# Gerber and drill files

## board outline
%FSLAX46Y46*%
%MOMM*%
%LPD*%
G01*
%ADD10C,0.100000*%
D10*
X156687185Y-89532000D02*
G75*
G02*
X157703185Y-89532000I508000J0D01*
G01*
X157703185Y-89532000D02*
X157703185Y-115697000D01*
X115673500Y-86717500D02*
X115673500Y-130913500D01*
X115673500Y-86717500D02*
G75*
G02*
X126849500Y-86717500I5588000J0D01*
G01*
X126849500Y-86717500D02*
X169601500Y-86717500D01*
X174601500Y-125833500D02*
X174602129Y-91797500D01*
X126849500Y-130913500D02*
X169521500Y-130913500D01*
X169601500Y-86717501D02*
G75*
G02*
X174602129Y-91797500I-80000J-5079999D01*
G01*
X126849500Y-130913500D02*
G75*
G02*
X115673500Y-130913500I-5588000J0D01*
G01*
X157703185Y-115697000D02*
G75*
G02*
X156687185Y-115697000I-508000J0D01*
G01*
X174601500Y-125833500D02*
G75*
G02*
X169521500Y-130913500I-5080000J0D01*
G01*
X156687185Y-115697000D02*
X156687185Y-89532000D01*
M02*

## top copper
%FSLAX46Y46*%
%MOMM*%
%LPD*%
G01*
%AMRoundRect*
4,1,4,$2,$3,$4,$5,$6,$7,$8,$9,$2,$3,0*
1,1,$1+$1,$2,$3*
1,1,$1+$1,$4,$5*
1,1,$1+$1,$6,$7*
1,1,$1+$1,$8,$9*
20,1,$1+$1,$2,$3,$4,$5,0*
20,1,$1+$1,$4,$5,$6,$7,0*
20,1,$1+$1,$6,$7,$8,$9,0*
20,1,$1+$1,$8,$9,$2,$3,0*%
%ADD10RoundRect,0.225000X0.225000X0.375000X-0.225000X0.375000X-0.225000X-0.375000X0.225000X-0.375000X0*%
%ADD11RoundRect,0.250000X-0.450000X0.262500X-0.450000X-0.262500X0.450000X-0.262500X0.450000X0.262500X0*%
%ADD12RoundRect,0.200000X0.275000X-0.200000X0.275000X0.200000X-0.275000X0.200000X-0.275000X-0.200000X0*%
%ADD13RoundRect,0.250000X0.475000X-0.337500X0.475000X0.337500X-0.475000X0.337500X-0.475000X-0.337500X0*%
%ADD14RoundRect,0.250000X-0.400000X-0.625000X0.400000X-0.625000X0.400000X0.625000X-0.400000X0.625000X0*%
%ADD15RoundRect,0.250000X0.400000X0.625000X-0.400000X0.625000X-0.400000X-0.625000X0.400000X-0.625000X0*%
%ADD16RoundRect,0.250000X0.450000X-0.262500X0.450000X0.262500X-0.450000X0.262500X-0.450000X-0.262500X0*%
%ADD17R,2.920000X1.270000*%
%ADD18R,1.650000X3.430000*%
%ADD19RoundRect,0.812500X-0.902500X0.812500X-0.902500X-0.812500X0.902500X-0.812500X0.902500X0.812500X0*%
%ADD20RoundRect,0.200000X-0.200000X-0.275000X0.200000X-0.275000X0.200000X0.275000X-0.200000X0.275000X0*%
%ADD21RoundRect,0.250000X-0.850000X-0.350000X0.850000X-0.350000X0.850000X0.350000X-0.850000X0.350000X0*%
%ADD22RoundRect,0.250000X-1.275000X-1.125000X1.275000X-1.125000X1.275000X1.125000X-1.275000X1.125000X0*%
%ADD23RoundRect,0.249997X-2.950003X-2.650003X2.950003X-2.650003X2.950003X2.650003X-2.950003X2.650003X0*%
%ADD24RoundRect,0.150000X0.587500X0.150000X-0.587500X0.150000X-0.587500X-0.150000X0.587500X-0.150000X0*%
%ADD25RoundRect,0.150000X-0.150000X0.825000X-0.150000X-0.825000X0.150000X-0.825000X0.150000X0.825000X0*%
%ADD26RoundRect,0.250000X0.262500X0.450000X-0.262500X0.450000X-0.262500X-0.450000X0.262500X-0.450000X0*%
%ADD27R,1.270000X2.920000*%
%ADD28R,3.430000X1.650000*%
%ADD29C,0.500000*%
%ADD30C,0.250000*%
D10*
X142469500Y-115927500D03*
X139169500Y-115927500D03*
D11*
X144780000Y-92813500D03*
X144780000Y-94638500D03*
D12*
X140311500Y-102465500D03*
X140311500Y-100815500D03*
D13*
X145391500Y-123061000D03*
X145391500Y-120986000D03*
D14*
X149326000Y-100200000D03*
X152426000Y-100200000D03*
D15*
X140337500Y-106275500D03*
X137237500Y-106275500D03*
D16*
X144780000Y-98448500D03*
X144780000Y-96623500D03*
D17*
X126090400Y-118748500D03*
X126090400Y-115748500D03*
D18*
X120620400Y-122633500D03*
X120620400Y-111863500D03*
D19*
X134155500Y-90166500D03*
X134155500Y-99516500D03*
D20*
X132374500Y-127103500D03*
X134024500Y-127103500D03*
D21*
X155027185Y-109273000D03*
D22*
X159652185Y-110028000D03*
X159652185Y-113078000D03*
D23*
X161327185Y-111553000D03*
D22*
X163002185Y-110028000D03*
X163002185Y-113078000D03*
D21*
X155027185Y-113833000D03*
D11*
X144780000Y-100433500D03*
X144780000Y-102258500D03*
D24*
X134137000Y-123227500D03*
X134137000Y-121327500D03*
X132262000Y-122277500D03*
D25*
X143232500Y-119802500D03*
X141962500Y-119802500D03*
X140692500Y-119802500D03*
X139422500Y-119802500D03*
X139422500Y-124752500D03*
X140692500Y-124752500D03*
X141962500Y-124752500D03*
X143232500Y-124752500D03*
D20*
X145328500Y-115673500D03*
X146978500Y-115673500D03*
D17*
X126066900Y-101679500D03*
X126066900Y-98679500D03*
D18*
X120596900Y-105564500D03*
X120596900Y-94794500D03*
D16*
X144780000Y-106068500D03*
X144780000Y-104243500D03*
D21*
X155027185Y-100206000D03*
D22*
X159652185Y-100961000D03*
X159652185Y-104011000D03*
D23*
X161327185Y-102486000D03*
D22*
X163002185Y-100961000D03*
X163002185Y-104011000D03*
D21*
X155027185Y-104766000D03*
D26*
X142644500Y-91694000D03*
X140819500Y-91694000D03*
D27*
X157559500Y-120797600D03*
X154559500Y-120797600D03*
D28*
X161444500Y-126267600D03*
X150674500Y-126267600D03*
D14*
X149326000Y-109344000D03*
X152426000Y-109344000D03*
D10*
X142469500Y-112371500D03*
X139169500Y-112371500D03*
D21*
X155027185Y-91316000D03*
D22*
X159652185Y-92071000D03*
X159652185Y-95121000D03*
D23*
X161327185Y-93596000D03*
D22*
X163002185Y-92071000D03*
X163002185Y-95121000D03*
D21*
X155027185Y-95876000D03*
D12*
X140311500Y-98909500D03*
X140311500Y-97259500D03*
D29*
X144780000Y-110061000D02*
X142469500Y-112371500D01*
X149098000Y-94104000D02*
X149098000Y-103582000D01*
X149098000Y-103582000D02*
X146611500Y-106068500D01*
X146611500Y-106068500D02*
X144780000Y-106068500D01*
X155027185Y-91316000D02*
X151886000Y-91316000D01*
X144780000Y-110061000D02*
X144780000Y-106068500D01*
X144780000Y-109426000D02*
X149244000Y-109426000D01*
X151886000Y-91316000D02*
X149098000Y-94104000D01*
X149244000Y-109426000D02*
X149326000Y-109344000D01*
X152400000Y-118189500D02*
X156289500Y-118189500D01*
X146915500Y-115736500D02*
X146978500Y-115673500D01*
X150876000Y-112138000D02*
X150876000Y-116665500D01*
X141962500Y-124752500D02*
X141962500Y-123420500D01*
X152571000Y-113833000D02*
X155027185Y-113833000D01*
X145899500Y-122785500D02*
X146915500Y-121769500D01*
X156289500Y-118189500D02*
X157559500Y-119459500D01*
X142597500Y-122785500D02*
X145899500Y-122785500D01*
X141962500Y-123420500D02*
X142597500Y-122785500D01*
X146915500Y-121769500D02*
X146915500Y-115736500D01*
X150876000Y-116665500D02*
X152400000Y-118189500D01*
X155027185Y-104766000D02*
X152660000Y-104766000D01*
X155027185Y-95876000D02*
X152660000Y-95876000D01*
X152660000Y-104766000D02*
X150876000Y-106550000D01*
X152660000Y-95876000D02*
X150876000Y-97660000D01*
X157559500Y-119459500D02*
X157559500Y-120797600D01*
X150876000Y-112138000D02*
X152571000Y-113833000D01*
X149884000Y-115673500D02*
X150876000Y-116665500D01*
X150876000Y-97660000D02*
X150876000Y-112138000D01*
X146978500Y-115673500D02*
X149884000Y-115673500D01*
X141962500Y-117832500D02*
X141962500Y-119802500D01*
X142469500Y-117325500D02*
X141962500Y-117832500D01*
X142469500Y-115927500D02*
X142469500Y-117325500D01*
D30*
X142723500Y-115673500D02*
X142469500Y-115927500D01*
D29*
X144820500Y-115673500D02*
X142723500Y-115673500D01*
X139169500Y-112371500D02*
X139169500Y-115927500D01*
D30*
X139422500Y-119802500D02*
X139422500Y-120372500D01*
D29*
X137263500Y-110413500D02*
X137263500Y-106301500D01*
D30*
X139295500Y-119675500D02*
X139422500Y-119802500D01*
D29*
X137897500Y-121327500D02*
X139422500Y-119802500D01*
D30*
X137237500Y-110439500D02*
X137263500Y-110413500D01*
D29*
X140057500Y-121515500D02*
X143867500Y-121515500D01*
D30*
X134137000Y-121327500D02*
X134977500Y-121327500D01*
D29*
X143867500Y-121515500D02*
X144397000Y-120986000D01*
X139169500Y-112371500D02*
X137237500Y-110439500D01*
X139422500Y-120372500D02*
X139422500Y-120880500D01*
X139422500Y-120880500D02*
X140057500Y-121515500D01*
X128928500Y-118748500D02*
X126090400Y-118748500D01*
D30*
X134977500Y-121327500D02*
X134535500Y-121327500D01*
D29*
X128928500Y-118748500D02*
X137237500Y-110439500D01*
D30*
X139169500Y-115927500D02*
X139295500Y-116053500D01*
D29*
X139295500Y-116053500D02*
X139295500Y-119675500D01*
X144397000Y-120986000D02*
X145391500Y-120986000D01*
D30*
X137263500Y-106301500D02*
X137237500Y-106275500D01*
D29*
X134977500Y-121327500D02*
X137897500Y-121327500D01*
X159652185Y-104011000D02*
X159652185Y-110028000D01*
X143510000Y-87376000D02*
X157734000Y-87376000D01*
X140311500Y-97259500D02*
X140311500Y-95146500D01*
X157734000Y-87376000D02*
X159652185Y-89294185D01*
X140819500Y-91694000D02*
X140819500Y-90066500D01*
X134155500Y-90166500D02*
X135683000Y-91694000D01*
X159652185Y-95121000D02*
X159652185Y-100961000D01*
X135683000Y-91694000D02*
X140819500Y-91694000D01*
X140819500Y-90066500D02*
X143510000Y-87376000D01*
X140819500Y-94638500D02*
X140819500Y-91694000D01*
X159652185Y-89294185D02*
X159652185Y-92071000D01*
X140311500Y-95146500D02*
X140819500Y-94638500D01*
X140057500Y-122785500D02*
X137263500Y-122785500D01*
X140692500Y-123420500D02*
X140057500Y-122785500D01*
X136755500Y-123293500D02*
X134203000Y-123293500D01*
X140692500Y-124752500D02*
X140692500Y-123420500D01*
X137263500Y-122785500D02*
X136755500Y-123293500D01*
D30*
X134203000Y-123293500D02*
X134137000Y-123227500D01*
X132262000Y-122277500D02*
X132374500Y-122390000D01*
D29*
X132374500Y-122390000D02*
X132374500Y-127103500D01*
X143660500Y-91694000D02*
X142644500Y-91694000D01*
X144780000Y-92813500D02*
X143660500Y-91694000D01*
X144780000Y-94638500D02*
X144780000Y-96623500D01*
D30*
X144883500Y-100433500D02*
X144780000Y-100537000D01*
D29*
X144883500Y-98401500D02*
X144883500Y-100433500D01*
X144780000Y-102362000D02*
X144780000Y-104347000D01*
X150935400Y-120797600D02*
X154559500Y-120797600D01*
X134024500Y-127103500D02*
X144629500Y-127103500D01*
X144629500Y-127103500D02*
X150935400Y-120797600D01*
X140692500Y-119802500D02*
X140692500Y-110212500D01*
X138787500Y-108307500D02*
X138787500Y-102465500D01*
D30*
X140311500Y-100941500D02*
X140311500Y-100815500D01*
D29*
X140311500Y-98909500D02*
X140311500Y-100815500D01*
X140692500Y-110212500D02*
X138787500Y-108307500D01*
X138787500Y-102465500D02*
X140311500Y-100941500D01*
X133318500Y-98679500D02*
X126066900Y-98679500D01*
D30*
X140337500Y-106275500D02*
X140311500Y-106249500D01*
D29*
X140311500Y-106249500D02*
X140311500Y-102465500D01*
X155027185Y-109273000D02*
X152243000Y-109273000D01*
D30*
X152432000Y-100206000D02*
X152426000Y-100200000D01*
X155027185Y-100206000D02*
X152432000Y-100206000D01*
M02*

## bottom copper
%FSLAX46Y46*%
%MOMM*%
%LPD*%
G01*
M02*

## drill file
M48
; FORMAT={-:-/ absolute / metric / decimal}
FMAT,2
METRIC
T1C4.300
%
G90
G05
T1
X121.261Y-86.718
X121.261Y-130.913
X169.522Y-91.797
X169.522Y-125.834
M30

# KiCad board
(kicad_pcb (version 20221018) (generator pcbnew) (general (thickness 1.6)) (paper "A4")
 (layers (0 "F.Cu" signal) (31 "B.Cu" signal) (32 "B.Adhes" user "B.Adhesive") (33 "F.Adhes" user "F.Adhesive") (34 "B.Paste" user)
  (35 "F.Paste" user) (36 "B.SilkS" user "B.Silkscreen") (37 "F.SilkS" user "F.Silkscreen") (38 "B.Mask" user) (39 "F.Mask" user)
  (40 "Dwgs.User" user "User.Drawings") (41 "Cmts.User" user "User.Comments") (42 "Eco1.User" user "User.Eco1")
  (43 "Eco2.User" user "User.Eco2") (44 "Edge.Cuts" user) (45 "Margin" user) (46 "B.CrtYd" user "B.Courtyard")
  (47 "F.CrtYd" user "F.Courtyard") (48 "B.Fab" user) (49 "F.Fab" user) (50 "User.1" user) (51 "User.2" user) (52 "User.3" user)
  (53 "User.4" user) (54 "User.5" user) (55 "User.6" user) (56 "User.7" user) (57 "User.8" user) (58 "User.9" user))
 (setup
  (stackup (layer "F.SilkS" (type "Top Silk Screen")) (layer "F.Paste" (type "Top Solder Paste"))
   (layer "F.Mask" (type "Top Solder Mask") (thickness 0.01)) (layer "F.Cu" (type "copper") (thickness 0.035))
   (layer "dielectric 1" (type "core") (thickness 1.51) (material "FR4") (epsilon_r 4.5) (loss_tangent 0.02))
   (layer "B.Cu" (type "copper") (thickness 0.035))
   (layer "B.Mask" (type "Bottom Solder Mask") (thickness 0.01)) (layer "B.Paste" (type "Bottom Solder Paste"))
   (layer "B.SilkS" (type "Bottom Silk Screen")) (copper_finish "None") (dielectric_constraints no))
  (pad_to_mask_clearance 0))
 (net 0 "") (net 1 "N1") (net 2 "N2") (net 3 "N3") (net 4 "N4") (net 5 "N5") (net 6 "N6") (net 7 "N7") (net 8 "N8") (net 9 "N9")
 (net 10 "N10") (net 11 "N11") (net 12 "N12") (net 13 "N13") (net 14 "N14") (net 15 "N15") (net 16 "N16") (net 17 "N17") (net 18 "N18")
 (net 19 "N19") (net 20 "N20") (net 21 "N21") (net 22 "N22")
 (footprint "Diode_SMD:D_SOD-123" (layer "F.Cu") (at 140.8195 115.9275 180)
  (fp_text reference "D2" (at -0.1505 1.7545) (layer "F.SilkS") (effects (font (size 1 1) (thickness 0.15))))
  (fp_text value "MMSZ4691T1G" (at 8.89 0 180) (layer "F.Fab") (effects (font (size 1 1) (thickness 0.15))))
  (pad "1" smd roundrect (at -1.65 0 180) (size 0.9 1.2) (layers "F.Cu" "F.Paste" "F.Mask") (roundrect_rratio 0.25) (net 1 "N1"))
  (pad "2" smd roundrect (at 1.65 0 180) (size 0.9 1.2) (layers "F.Cu" "F.Paste" "F.Mask") (roundrect_rratio 0.25) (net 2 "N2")))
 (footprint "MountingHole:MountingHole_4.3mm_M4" (layer "F.Cu") (at 169.5215 91.7975)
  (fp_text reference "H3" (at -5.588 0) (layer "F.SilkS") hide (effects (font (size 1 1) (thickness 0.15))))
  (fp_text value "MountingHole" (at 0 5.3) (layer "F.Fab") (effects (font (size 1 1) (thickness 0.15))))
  (pad "" np_thru_hole circle (at 0 0) (size 4.3 4.3) (drill 4.3) (layers "*.Cu" "*.Mask")))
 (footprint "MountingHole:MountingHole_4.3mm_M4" (layer "F.Cu") (at 121.2615 130.9135)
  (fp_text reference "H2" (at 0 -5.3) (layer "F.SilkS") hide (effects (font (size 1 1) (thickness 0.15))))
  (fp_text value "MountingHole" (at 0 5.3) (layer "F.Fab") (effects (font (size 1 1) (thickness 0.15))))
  (pad "" np_thru_hole circle (at 0 0) (size 4.3 4.3) (drill 4.3) (layers "*.Cu" "*.Mask")))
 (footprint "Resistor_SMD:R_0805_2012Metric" (layer "F.Cu") (at 144.78 93.726 -90)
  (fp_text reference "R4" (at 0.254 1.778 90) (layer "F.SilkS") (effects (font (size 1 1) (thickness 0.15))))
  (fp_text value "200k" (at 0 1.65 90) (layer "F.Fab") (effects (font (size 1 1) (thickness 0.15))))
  (pad "1" smd roundrect (at -0.9125 0 270) (size 1.025 1.4) (layers "F.Cu" "F.Paste" "F.Mask") (roundrect_rratio 0.243902) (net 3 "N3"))
  (pad "2" smd roundrect (at 0.9125 0 270) (size 1.025 1.4) (layers "F.Cu" "F.Paste" "F.Mask") (roundrect_rratio 0.243902) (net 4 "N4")))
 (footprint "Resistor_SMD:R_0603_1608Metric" (layer "F.Cu") (at 140.3115 101.6405 90)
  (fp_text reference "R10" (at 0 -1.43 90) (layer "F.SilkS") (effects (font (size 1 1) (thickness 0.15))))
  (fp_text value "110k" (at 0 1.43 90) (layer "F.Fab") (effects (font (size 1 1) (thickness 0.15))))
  (pad "1" smd roundrect (at -0.825 0 90) (size 0.8 0.95) (layers "F.Cu" "F.Paste" "F.Mask") (roundrect_rratio 0.25) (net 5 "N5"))
  (pad "2" smd roundrect (at 0.825 0 90) (size 0.8 0.95) (layers "F.Cu" "F.Paste" "F.Mask") (roundrect_rratio 0.25) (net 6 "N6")))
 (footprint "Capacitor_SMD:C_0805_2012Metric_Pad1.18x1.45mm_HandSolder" (layer "F.Cu") (at 145.3915 122.0235 90)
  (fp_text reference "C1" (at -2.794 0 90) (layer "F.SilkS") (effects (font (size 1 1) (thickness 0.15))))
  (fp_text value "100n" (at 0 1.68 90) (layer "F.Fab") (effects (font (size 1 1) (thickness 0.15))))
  (pad "1" smd roundrect (at -1.0375 0 90) (size 1.175 1.45) (layers "F.Cu" "F.Paste" "F.Mask") (roundrect_rratio 0.212766) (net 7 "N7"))
  (pad "2" smd roundrect (at 1.0375 0 90) (size 1.175 1.45) (layers "F.Cu" "F.Paste" "F.Mask") (roundrect_rratio 0.212766) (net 2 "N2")))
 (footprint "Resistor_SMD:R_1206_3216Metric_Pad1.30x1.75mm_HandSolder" (layer "F.Cu") (at 150.876 100.2)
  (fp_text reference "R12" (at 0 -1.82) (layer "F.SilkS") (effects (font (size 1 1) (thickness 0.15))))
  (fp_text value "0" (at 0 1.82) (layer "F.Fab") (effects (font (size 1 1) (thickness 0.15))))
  (pad "1" smd roundrect (at -1.55 0) (size 1.3 1.75) (layers "F.Cu" "F.Paste" "F.Mask") (roundrect_rratio 0.192308) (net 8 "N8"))
  (pad "2" smd roundrect (at 1.55 0) (size 1.3 1.75) (layers "F.Cu" "F.Paste" "F.Mask") (roundrect_rratio 0.192308) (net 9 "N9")))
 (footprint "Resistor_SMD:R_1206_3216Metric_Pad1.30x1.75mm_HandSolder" (layer "F.Cu") (at 138.7875 106.2755 180)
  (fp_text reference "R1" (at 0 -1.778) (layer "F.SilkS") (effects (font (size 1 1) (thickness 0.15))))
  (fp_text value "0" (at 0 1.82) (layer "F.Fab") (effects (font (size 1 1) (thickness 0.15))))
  (pad "1" smd roundrect (at -1.55 0 180) (size 1.3 1.75) (layers "F.Cu" "F.Paste" "F.Mask") (roundrect_rratio 0.192308) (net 5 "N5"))
  (pad "2" smd roundrect (at 1.55 0 180) (size 1.3 1.75) (layers "F.Cu" "F.Paste" "F.Mask") (roundrect_rratio 0.192308) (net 2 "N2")))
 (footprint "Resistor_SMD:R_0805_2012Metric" (layer "F.Cu") (at 144.78 97.536 90)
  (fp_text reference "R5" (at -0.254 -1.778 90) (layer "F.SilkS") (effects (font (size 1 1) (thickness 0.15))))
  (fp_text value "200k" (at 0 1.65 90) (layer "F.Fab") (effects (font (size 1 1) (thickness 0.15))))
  (pad "1" smd roundrect (at -0.9125 0 90) (size 1.025 1.4) (layers "F.Cu" "F.Paste" "F.Mask") (roundrect_rratio 0.243902) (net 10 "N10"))
  (pad "2" smd roundrect (at 0.9125 0 90) (size 1.025 1.4) (layers "F.Cu" "F.Paste" "F.Mask") (roundrect_rratio 0.243902) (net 4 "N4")))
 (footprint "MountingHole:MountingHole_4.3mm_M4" (layer "F.Cu") (at 169.5215 125.8335)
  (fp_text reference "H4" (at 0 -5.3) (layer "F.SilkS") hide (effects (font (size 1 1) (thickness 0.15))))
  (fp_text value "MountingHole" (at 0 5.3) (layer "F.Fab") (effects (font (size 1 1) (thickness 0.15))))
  (pad "" np_thru_hole circle (at 0 0) (size 4.3 4.3) (drill 4.3) (layers "*.Cu" "*.Mask")))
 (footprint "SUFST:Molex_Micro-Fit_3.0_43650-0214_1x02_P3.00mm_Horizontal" (layer "F.Cu") (at 126.0904 117.2485 -90)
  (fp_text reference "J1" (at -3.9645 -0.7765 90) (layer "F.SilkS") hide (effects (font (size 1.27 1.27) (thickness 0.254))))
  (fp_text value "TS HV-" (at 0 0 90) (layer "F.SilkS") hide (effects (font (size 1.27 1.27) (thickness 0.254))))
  (pad "1" smd rect (at 1.5 0 270) (size 1.27 2.92) (layers "F.Cu" "F.Paste" "F.Mask") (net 2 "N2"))
  (pad "2" smd rect (at -1.5 0 270) (size 1.27 2.92) (layers "F.Cu" "F.Paste" "F.Mask") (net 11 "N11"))
  (pad "3" smd rect (at 5.385 5.47) (size 1.65 3.43) (layers "F.Cu" "F.Paste" "F.Mask"))
  (pad "4" smd rect (at -5.385 5.47) (size 1.65 3.43) (layers "F.Cu" "F.Paste" "F.Mask")))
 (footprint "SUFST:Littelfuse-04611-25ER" (layer "F.Cu") (at 134.2155 94.5915 -90)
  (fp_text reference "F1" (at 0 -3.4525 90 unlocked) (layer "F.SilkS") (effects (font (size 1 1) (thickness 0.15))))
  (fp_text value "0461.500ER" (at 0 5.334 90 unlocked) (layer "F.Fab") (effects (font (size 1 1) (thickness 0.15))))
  (pad "1" smd roundrect (at -4.425 0.06 270) (size 3.25 3.43) (layers "F.Cu" "F.Paste" "F.Mask") (roundrect_rratio 0.25) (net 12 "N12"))
  (pad "2" smd roundrect (at 4.925 0.06 270) (size 3.25 3.43) (layers "F.Cu" "F.Paste" "F.Mask") (roundrect_rratio 0.25) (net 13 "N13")))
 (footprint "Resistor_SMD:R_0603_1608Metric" (layer "F.Cu") (at 133.1995 127.1035)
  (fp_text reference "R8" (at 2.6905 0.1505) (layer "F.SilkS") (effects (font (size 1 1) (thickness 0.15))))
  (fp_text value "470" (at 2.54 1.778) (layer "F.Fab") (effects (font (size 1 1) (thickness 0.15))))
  (pad "1" smd roundrect (at -0.825 0) (size 0.8 0.95) (layers "F.Cu" "F.Paste" "F.Mask") (roundrect_rratio 0.25) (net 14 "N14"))
  (pad "2" smd roundrect (at 0.825 0) (size 0.8 0.95) (layers "F.Cu" "F.Paste" "F.Mask") (roundrect_rratio 0.25) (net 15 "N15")))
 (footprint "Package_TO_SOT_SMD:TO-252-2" (layer "F.Cu") (at 160.067185 111.553)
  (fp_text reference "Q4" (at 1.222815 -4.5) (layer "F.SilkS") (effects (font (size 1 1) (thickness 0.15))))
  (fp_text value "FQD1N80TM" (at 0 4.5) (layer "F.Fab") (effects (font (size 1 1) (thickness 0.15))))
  (pad "1" smd roundrect (at -5.04 -2.28) (size 2.2 1.2) (layers "F.Cu" "F.Paste" "F.Mask") (roundrect_rratio 0.208333) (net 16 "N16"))
  (pad "2" smd roundrect (at -0.415 -1.525) (size 3.05 2.75) (layers "F.Cu" "F.Paste") (roundrect_rratio 0.090909) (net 12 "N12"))
  (pad "2" smd roundrect (at -0.415 1.525) (size 3.05 2.75) (layers "F.Cu" "F.Paste") (roundrect_rratio 0.090909) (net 12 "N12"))
  (pad "2" smd roundrect (at 1.26 0) (size 6.4 5.8) (layers "F.Cu" "F.Mask") (roundrect_rratio 0.043103) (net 12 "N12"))
  (pad "2" smd roundrect (at 2.935 -1.525) (size 3.05 2.75) (layers "F.Cu" "F.Paste") (roundrect_rratio 0.090909) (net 12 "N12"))
  (pad "2" smd roundrect (at 2.935 1.525) (size 3.05 2.75) (layers "F.Cu" "F.Paste") (roundrect_rratio 0.090909) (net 12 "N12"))
  (pad "3" smd roundrect (at -5.04 2.28) (size 2.2 1.2) (layers "F.Cu" "F.Paste" "F.Mask") (roundrect_rratio 0.208333) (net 7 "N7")))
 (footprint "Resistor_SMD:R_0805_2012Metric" (layer "F.Cu") (at 144.78 101.346 -90)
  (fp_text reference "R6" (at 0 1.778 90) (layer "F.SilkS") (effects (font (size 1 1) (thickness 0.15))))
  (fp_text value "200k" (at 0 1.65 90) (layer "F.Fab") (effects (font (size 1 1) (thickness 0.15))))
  (pad "1" smd roundrect (at -0.9125 0 270) (size 1.025 1.4) (layers "F.Cu" "F.Paste" "F.Mask") (roundrect_rratio 0.243902) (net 10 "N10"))
  (pad "2" smd roundrect (at 0.9125 0 270) (size 1.025 1.4) (layers "F.Cu" "F.Paste" "F.Mask") (roundrect_rratio 0.243902) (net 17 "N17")))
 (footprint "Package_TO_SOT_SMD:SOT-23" (layer "F.Cu") (at 133.1995 122.2775 180)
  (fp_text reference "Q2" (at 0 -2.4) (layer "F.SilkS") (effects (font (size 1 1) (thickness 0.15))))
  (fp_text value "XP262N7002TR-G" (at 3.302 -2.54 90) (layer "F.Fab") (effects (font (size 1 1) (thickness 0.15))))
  (pad "1" smd roundrect (at -0.9375 -0.95 180) (size 1.475 0.6) (layers "F.Cu" "F.Paste" "F.Mask") (roundrect_rratio 0.25) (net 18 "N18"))
  (pad "2" smd roundrect (at -0.9375 0.95 180) (size 1.475 0.6) (layers "F.Cu" "F.Paste" "F.Mask") (roundrect_rratio 0.25) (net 2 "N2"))
  (pad "3" smd roundrect (at 0.9375 0 180) (size 1.475 0.6) (layers "F.Cu" "F.Paste" "F.Mask") (roundrect_rratio 0.25) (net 14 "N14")))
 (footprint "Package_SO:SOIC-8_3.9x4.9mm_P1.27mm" (layer "F.Cu") (at 141.3275 122.2775 -90)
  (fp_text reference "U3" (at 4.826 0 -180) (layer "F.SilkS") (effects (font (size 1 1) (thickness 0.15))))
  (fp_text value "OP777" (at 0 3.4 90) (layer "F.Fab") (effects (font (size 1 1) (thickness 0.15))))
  (pad "1" smd roundrect (at -2.475 -1.905 270) (size 1.95 0.6) (layers "F.Cu" "F.Paste" "F.Mask") (roundrect_rratio 0.25) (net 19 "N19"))
  (pad "2" smd roundrect (at -2.475 -0.635 270) (size 1.95 0.6) (layers "F.Cu" "F.Paste" "F.Mask") (roundrect_rratio 0.25) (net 1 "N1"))
  (pad "3" smd roundrect (at -2.475 0.635 270) (size 1.95 0.6) (layers "F.Cu" "F.Paste" "F.Mask") (roundrect_rratio 0.25) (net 6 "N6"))
  (pad "4" smd roundrect (at -2.475 1.905 270) (size 1.95 0.6) (layers "F.Cu" "F.Paste" "F.Mask") (roundrect_rratio 0.25) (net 2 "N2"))
  (pad "5" smd roundrect (at 2.475 1.905 270) (size 1.95 0.6) (layers "F.Cu" "F.Paste" "F.Mask") (roundrect_rratio 0.25) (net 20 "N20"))
  (pad "6" smd roundrect (at 2.475 0.635 270) (size 1.95 0.6) (layers "F.Cu" "F.Paste" "F.Mask") (roundrect_rratio 0.25) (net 18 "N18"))
  (pad "7" smd roundrect (at 2.475 -0.635 270) (size 1.95 0.6) (layers "F.Cu" "F.Paste" "F.Mask") (roundrect_rratio 0.25) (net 7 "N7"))
  (pad "8" smd roundrect (at 2.475 -1.905 270) (size 1.95 0.6) (layers "F.Cu" "F.Paste" "F.Mask") (roundrect_rratio 0.25) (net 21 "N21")))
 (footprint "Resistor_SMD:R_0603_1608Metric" (layer "F.Cu") (at 146.1535 115.6735)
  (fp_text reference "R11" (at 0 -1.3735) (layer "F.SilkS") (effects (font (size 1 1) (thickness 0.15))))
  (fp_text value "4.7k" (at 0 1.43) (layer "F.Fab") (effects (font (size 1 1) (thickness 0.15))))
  (pad "1" smd roundrect (at -0.825 0) (size 0.8 0.95) (layers "F.Cu" "F.Paste" "F.Mask") (roundrect_rratio 0.25) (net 1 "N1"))
  (pad "2" smd roundrect (at 0.825 0) (size 0.8 0.95) (layers "F.Cu" "F.Paste" "F.Mask") (roundrect_rratio 0.25) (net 7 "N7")))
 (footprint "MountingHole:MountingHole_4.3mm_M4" (layer "F.Cu") (at 121.2615 86.7175)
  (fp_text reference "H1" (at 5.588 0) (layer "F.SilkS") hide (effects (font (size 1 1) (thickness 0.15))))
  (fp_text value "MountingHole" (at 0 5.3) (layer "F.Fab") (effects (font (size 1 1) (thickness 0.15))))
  (pad "" np_thru_hole circle (at 0 0) (size 4.3 4.3) (drill 4.3) (layers "*.Cu" "*.Mask")))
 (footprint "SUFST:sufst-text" (layer "F.Cu") (at 168.402 108.712 90)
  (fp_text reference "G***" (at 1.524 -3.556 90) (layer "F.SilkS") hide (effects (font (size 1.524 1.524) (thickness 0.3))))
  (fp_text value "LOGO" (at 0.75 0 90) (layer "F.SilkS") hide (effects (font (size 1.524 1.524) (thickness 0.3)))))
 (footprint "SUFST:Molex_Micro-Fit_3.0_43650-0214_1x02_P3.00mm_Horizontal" (layer "F.Cu") (at 126.0669 100.1795 -90)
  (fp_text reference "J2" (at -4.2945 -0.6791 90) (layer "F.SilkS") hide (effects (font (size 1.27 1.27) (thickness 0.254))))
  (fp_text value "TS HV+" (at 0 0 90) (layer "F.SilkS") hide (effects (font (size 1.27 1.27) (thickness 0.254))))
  (pad "1" smd rect (at 1.5 0 270) (size 1.27 2.92) (layers "F.Cu" "F.Paste" "F.Mask") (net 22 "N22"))
  (pad "2" smd rect (at -1.5 0 270) (size 1.27 2.92) (layers "F.Cu" "F.Paste" "F.Mask") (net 13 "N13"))
  (pad "3" smd rect (at 5.385 5.47) (size 1.65 3.43) (layers "F.Cu" "F.Paste" "F.Mask"))
  (pad "4" smd rect (at -5.385 5.47) (size 1.65 3.43) (layers "F.Cu" "F.Paste" "F.Mask")))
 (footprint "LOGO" (layer "F.Cu") (at 131.064 113.792 90)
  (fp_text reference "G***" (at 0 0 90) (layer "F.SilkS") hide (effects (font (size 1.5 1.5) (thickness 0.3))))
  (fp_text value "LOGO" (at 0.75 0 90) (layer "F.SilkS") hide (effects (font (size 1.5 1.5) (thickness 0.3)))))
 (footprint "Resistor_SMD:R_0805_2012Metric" (layer "F.Cu") (at 144.78 105.156 90)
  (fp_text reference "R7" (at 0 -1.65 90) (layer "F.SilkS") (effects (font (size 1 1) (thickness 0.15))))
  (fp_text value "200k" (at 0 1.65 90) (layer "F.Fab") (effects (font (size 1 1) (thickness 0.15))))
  (pad "1" smd roundrect (at -0.9125 0 90) (size 1.025 1.4) (layers "F.Cu" "F.Paste" "F.Mask") (roundrect_rratio 0.243902) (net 8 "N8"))
  (pad "2" smd roundrect (at 0.9125 0 90) (size 1.025 1.4) (layers "F.Cu" "F.Paste" "F.Mask") (roundrect_rratio 0.243902) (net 17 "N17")))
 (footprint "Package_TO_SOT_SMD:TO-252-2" (layer "F.Cu") (at 160.067185 102.486)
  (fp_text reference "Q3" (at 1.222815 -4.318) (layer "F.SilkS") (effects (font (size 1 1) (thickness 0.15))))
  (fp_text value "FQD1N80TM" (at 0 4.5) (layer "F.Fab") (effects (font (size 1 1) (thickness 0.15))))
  (pad "1" smd roundrect (at -5.04 -2.28) (size 2.2 1.2) (layers "F.Cu" "F.Paste" "F.Mask") (roundrect_rratio 0.208333) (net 9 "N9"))
  (pad "2" smd roundrect (at -0.415 -1.525) (size 3.05 2.75) (layers "F.Cu" "F.Paste") (roundrect_rratio 0.090909) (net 12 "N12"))
  (pad "2" smd roundrect (at -0.415 1.525) (size 3.05 2.75) (layers "F.Cu" "F.Paste") (roundrect_rratio 0.090909) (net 12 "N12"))
  (pad "2" smd roundrect (at 1.26 0) (size 6.4 5.8) (layers "F.Cu" "F.Mask") (roundrect_rratio 0.043103) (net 12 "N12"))
  (pad "2" smd roundrect (at 2.935 -1.525) (size 3.05 2.75) (layers "F.Cu" "F.Paste") (roundrect_rratio 0.090909) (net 12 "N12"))
  (pad "2" smd roundrect (at 2.935 1.525) (size 3.05 2.75) (layers "F.Cu" "F.Paste") (roundrect_rratio 0.090909) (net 12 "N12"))
  (pad "3" smd roundrect (at -5.04 2.28) (size 2.2 1.2) (layers "F.Cu" "F.Paste" "F.Mask") (roundrect_rratio 0.208333) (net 7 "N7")))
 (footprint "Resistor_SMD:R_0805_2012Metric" (layer "F.Cu") (at 141.732 91.694 180)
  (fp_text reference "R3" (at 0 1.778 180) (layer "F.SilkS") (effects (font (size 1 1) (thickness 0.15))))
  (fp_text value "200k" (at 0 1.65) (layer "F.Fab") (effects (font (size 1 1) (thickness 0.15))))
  (pad "1" smd roundrect (at -0.9125 0 180) (size 1.025 1.4) (layers "F.Cu" "F.Paste" "F.Mask") (roundrect_rratio 0.243902) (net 3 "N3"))
  (pad "2" smd roundrect (at 0.9125 0 180) (size 1.025 1.4) (layers "F.Cu" "F.Paste" "F.Mask") (roundrect_rratio 0.243902) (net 12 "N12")))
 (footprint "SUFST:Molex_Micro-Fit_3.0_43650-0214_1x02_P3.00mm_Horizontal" (layer "F.Cu") (at 156.0595 120.7976)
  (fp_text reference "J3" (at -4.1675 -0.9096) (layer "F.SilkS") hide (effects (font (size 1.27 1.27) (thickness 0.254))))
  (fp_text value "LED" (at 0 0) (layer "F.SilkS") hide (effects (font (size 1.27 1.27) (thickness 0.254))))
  (pad "1" smd rect (at 1.5 0) (size 1.27 2.92) (layers "F.Cu" "F.Paste" "F.Mask") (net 7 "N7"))
  (pad "2" smd rect (at -1.5 0) (size 1.27 2.92) (layers "F.Cu" "F.Paste" "F.Mask") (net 15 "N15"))
  (pad "3" smd rect (at 5.385 5.47 90) (size 1.65 3.43) (layers "F.Cu" "F.Paste" "F.Mask"))
  (pad "4" smd rect (at -5.385 5.47 90) (size 1.65 3.43) (layers "F.Cu" "F.Paste" "F.Mask")))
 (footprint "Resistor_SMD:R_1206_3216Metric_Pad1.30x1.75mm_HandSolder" (layer "F.Cu") (at 150.876 109.344)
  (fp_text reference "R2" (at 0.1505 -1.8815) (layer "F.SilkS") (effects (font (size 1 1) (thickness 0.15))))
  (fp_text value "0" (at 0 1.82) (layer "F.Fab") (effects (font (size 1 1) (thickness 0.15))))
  (pad "1" smd roundrect (at -1.55 0) (size 1.3 1.75) (layers "F.Cu" "F.Paste" "F.Mask") (roundrect_rratio 0.192308) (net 8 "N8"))
  (pad "2" smd roundrect (at 1.55 0) (size 1.3 1.75) (layers "F.Cu" "F.Paste" "F.Mask") (roundrect_rratio 0.192308) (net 16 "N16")))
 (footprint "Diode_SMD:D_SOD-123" (layer "F.Cu") (at 140.8195 112.3715 180)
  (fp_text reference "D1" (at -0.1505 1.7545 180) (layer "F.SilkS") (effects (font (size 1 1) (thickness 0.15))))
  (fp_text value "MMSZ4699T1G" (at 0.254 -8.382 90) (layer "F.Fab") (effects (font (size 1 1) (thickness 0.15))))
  (pad "1" smd roundrect (at -1.65 0 180) (size 0.9 1.2) (layers "F.Cu" "F.Paste" "F.Mask") (roundrect_rratio 0.25) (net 8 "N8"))
  (pad "2" smd roundrect (at 1.65 0 180) (size 0.9 1.2) (layers "F.Cu" "F.Paste" "F.Mask") (roundrect_rratio 0.25) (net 2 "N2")))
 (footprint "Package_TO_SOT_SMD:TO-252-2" (layer "F.Cu") (at 160.067185 93.596)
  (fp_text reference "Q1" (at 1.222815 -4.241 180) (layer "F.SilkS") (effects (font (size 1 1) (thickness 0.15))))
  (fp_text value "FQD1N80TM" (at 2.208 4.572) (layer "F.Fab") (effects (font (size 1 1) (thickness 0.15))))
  (pad "1" smd roundrect (at -5.04 -2.28) (size 2.2 1.2) (layers "F.Cu" "F.Paste" "F.Mask") (roundrect_rratio 0.208333) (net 8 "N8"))
  (pad "2" smd roundrect (at -0.415 -1.525) (size 3.05 2.75) (layers "F.Cu" "F.Paste") (roundrect_rratio 0.090909) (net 12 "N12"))
  (pad "2" smd roundrect (at -0.415 1.525) (size 3.05 2.75) (layers "F.Cu" "F.Paste") (roundrect_rratio 0.090909) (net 12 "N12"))
  (pad "2" smd roundrect (at 1.26 0) (size 6.4 5.8) (layers "F.Cu" "F.Mask") (roundrect_rratio 0.043103) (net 12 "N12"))
  (pad "2" smd roundrect (at 2.935 -1.525) (size 3.05 2.75) (layers "F.Cu" "F.Paste") (roundrect_rratio 0.090909) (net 12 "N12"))
  (pad "2" smd roundrect (at 2.935 1.525) (size 3.05 2.75) (layers "F.Cu" "F.Paste") (roundrect_rratio 0.090909) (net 12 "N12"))
  (pad "3" smd roundrect (at -5.04 2.28) (size 2.2 1.2) (layers "F.Cu" "F.Paste" "F.Mask") (roundrect_rratio 0.208333) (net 7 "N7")))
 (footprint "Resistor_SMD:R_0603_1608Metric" (layer "F.Cu") (at 140.3115 98.0845 90)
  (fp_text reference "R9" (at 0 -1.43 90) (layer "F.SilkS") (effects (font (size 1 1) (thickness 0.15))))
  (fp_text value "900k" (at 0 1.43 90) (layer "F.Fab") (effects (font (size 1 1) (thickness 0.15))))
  (pad "1" smd roundrect (at -0.825 0 90) (size 0.8 0.95) (layers "F.Cu" "F.Paste" "F.Mask") (roundrect_rratio 0.25) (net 6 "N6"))
  (pad "2" smd roundrect (at 0.825 0 90) (size 0.8 0.95) (layers "F.Cu" "F.Paste" "F.Mask") (roundrect_rratio 0.25) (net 12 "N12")))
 (gr_arc (start 156.687185 89.532) (mid 157.195185 89.024) (end 157.703185 89.532) (stroke (width 0.1) (type default)) (layer "Edge.Cuts"))
 (gr_line (start 157.703185 89.532) (end 157.703185 115.697) (stroke (width 0.1) (type default)) (layer "Edge.Cuts"))
 (gr_line (start 115.6735 86.7175) (end 115.6735 130.9135) (stroke (width 0.1) (type default)) (layer "Edge.Cuts"))
 (gr_arc (start 115.6735 86.7175) (mid 121.2615 81.1295) (end 126.8495 86.7175) (stroke (width 0.1) (type default)) (layer "Edge.Cuts"))
 (gr_line (start 126.8495 86.7175) (end 169.6015 86.7175) (stroke (width 0.1) (type default)) (layer "Edge.Cuts"))
 (gr_line (start 174.6015 125.8335) (end 174.602129 91.7975) (stroke (width 0.1) (type default)) (layer "Edge.Cuts"))
 (gr_line (start 126.8495 130.9135) (end 169.5215 130.9135) (stroke (width 0.1) (type default)) (layer "Edge.Cuts"))
 (gr_arc (start 169.6015 86.717501) (mid 173.142221 88.233349) (end 174.602129 91.7975) (stroke (width 0.1) (type default))
  (layer "Edge.Cuts"))
 (gr_arc (start 126.8495 130.9135) (mid 121.2615 136.5015) (end 115.6735 130.9135) (stroke (width 0.1) (type default)) (layer "Edge.Cuts"))
 (gr_arc (start 157.703185 115.697) (mid 157.195185 116.205) (end 156.687185 115.697) (stroke (width 0.1) (type default))
  (layer "Edge.Cuts"))
 (gr_arc (start 174.6015 125.8335) (mid 173.113602 129.425602) (end 169.5215 130.9135) (stroke (width 0.1) (type default))
  (layer "Edge.Cuts"))
 (gr_line (start 156.687185 115.697) (end 156.687185 89.532) (stroke (width 0.1) (type default)) (layer "Edge.Cuts"))
 (segment (start 144.78 110.061) (end 142.4695 112.3715) (width 0.5) (layer "F.Cu") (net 8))
 (segment (start 149.098 94.104) (end 149.098 103.582) (width 0.5) (layer "F.Cu") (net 8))
 (segment (start 149.098 103.582) (end 146.6115 106.0685) (width 0.5) (layer "F.Cu") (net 8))
 (segment (start 146.6115 106.0685) (end 144.78 106.0685) (width 0.5) (layer "F.Cu") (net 8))
 (segment (start 155.027185 91.316) (end 151.886 91.316) (width 0.5) (layer "F.Cu") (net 8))
 (segment (start 144.78 110.061) (end 144.78 106.0685) (width 0.5) (layer "F.Cu") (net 8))
 (segment (start 144.78 109.426) (end 149.244 109.426) (width 0.5) (layer "F.Cu") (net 8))
 (segment (start 151.886 91.316) (end 149.098 94.104) (width 0.5) (layer "F.Cu") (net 8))
 (segment (start 149.244 109.426) (end 149.326 109.344) (width 0.5) (layer "F.Cu") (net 8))
 (segment (start 152.4 118.1895) (end 156.2895 118.1895) (width 0.5) (layer "F.Cu") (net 7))
 (segment (start 146.9155 115.7365) (end 146.9785 115.6735) (width 0.5) (layer "F.Cu") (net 7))
 (segment (start 150.876 112.138) (end 150.876 116.6655) (width 0.5) (layer "F.Cu") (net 7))
 (segment (start 141.9625 124.7525) (end 141.9625 123.4205) (width 0.5) (layer "F.Cu") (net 7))
 (segment (start 152.571 113.833) (end 155.027185 113.833) (width 0.5) (layer "F.Cu") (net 7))
 (segment (start 145.8995 122.7855) (end 146.9155 121.7695) (width 0.5) (layer "F.Cu") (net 7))
 (segment (start 156.2895 118.1895) (end 157.5595 119.4595) (width 0.5) (layer "F.Cu") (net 7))
 (segment (start 142.5975 122.7855) (end 145.8995 122.7855) (width 0.5) (layer "F.Cu") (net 7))
 (segment (start 141.9625 123.4205) (end 142.5975 122.7855) (width 0.5) (layer "F.Cu") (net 7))
 (segment (start 146.9155 121.7695) (end 146.9155 115.7365) (width 0.5) (layer "F.Cu") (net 7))
 (segment (start 150.876 116.6655) (end 152.4 118.1895) (width 0.5) (layer "F.Cu") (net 7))
 (segment (start 155.027185 104.766) (end 152.66 104.766) (width 0.5) (layer "F.Cu") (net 7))
 (segment (start 155.027185 95.876) (end 152.66 95.876) (width 0.5) (layer "F.Cu") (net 7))
 (segment (start 152.66 104.766) (end 150.876 106.55) (width 0.5) (layer "F.Cu") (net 7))
 (segment (start 152.66 95.876) (end 150.876 97.66) (width 0.5) (layer "F.Cu") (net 7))
 (segment (start 157.5595 119.4595) (end 157.5595 120.7976) (width 0.5) (layer "F.Cu") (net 7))
 (segment (start 150.876 112.138) (end 152.571 113.833) (width 0.5) (layer "F.Cu") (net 7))
 (segment (start 149.884 115.6735) (end 150.876 116.6655) (width 0.5) (layer "F.Cu") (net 7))
 (segment (start 150.876 97.66) (end 150.876 112.138) (width 0.5) (layer "F.Cu") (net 7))
 (segment (start 146.9785 115.6735) (end 149.884 115.6735) (width 0.5) (layer "F.Cu") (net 7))
 (segment (start 141.9625 117.8325) (end 141.9625 119.8025) (width 0.5) (layer "F.Cu") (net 1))
 (segment (start 142.4695 117.3255) (end 141.9625 117.8325) (width 0.5) (layer "F.Cu") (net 1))
 (segment (start 142.4695 115.9275) (end 142.4695 117.3255) (width 0.5) (layer "F.Cu") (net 1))
 (segment (start 142.7235 115.6735) (end 142.4695 115.9275) (width 0.25) (layer "F.Cu") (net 1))
 (segment (start 144.8205 115.6735) (end 142.7235 115.6735) (width 0.5) (layer "F.Cu") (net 1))
 (segment (start 139.1695 112.3715) (end 139.1695 115.9275) (width 0.5) (layer "F.Cu") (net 2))
 (segment (start 139.4225 119.8025) (end 139.4225 120.3725) (width 0.25) (layer "F.Cu") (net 2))
 (segment (start 137.2635 110.4135) (end 137.2635 106.3015) (width 0.5) (layer "F.Cu") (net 2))
 (segment (start 139.2955 119.6755) (end 139.4225 119.8025) (width 0.25) (layer "F.Cu") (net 2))
 (segment (start 137.8975 121.3275) (end 139.4225 119.8025) (width 0.5) (layer "F.Cu") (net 2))
 (segment (start 137.2375 110.4395) (end 137.2635 110.4135) (width 0.25) (layer "F.Cu") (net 2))
 (segment (start 140.0575 121.5155) (end 143.8675 121.5155) (width 0.5) (layer "F.Cu") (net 2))
 (segment (start 134.137 121.3275) (end 134.9775 121.3275) (width 0.25) (layer "F.Cu") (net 2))
 (segment (start 143.8675 121.5155) (end 144.397 120.986) (width 0.5) (layer "F.Cu") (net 2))
 (segment (start 139.1695 112.3715) (end 137.2375 110.4395) (width 0.5) (layer "F.Cu") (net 2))
 (segment (start 139.4225 120.3725) (end 139.4225 120.8805) (width 0.5) (layer "F.Cu") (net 2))
 (segment (start 139.4225 120.8805) (end 140.0575 121.5155) (width 0.5) (layer "F.Cu") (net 2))
 (segment (start 128.9285 118.7485) (end 126.0904 118.7485) (width 0.5) (layer "F.Cu") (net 2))
 (segment (start 134.9775 121.3275) (end 134.5355 121.3275) (width 0.25) (layer "F.Cu") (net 2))
 (segment (start 128.9285 118.7485) (end 137.2375 110.4395) (width 0.5) (layer "F.Cu") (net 2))
 (segment (start 139.1695 115.9275) (end 139.2955 116.0535) (width 0.25) (layer "F.Cu") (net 2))
 (segment (start 139.2955 116.0535) (end 139.2955 119.6755) (width 0.5) (layer "F.Cu") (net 2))
 (segment (start 144.397 120.986) (end 145.3915 120.986) (width 0.5) (layer "F.Cu") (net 2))
 (segment (start 137.2635 106.3015) (end 137.2375 106.2755) (width 0.25) (layer "F.Cu") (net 2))
 (segment (start 134.9775 121.3275) (end 137.8975 121.3275) (width 0.5) (layer "F.Cu") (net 2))
 (segment (start 159.652185 104.011) (end 159.652185 110.028) (width 0.5) (layer "F.Cu") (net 12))
 (segment (start 143.51 87.376) (end 157.734 87.376) (width 0.5) (layer "F.Cu") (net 12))
 (segment (start 140.3115 97.2595) (end 140.3115 95.1465) (width 0.5) (layer "F.Cu") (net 12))
 (segment (start 157.734 87.376) (end 159.652185 89.294185) (width 0.5) (layer "F.Cu") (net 12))
 (segment (start 140.8195 91.694) (end 140.8195 90.0665) (width 0.5) (layer "F.Cu") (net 12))
 (segment (start 134.1555 90.1665) (end 135.683 91.694) (width 0.5) (layer "F.Cu") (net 12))
 (segment (start 159.652185 95.121) (end 159.652185 100.961) (width 0.5) (layer "F.Cu") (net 12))
 (segment (start 135.683 91.694) (end 140.8195 91.694) (width 0.5) (layer "F.Cu") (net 12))
 (segment (start 140.8195 90.0665) (end 143.51 87.376) (width 0.5) (layer "F.Cu") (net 12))
 (segment (start 140.8195 94.6385) (end 140.8195 91.694) (width 0.5) (layer "F.Cu") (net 12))
 (segment (start 159.652185 89.294185) (end 159.652185 92.071) (width 0.5) (layer "F.Cu") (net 12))
 (segment (start 140.3115 95.1465) (end 140.8195 94.6385) (width 0.5) (layer "F.Cu") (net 12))
 (segment (start 140.0575 122.7855) (end 137.2635 122.7855) (width 0.5) (layer "F.Cu") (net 18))
 (segment (start 140.6925 123.4205) (end 140.0575 122.7855) (width 0.5) (layer "F.Cu") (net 18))
 (segment (start 136.7555 123.2935) (end 134.203 123.2935) (width 0.5) (layer "F.Cu") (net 18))
 (segment (start 140.6925 124.7525) (end 140.6925 123.4205) (width 0.5) (layer "F.Cu") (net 18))
 (segment (start 137.2635 122.7855) (end 136.7555 123.2935) (width 0.5) (layer "F.Cu") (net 18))
 (segment (start 134.203 123.2935) (end 134.137 123.2275) (width 0.25) (layer "F.Cu") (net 18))
 (segment (start 132.262 122.2775) (end 132.3745 122.39) (width 0.25) (layer "F.Cu") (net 14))
 (segment (start 132.3745 122.39) (end 132.3745 127.1035) (width 0.5) (layer "F.Cu") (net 14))
 (segment (start 143.6605 91.694) (end 142.6445 91.694) (width 0.5) (layer "F.Cu") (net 3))
 (segment (start 144.78 92.8135) (end 143.6605 91.694) (width 0.5) (layer "F.Cu") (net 3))
 (segment (start 144.78 94.6385) (end 144.78 96.6235) (width 0.5) (layer "F.Cu") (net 4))
 (segment (start 144.8835 100.4335) (end 144.78 100.537) (width 0.25) (layer "F.Cu") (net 10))
 (segment (start 144.8835 98.4015) (end 144.8835 100.4335) (width 0.5) (layer "F.Cu") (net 10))
 (segment (start 144.78 102.362) (end 144.78 104.347) (width 0.5) (layer "F.Cu") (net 17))
 (segment (start 150.9354 120.7976) (end 154.5595 120.7976) (width 0.5) (layer "F.Cu") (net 15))
 (segment (start 134.0245 127.1035) (end 144.6295 127.1035) (width 0.5) (layer "F.Cu") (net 15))
 (segment (start 144.6295 127.1035) (end 150.9354 120.7976) (width 0.5) (layer "F.Cu") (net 15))
 (segment (start 140.6925 119.8025) (end 140.6925 110.2125) (width 0.5) (layer "F.Cu") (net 6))
 (segment (start 138.7875 108.3075) (end 138.7875 102.4655) (width 0.5) (layer "F.Cu") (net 6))
 (segment (start 140.3115 100.9415) (end 140.3115 100.8155) (width 0.25) (layer "F.Cu") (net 6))
 (segment (start 140.3115 98.9095) (end 140.3115 100.8155) (width 0.5) (layer "F.Cu") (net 6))
 (segment (start 140.6925 110.2125) (end 138.7875 108.3075) (width 0.5) (layer "F.Cu") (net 6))
 (segment (start 138.7875 102.4655) (end 140.3115 100.9415) (width 0.5) (layer "F.Cu") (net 6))
 (segment (start 133.3185 98.6795) (end 126.0669 98.6795) (width 0.5) (layer "F.Cu") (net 13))
 (segment (start 140.3375 106.2755) (end 140.3115 106.2495) (width 0.25) (layer "F.Cu") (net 5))
 (segment (start 140.3115 106.2495) (end 140.3115 102.4655) (width 0.5) (layer "F.Cu") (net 5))
 (segment (start 155.027185 109.273) (end 152.243 109.273) (width 0.5) (layer "F.Cu") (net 16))
 (segment (start 152.432 100.206) (end 152.426 100.2) (width 0.25) (layer "F.Cu") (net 9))
 (segment (start 155.027185 100.206) (end 152.432 100.206) (width 0.25) (layer "F.Cu") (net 9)))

